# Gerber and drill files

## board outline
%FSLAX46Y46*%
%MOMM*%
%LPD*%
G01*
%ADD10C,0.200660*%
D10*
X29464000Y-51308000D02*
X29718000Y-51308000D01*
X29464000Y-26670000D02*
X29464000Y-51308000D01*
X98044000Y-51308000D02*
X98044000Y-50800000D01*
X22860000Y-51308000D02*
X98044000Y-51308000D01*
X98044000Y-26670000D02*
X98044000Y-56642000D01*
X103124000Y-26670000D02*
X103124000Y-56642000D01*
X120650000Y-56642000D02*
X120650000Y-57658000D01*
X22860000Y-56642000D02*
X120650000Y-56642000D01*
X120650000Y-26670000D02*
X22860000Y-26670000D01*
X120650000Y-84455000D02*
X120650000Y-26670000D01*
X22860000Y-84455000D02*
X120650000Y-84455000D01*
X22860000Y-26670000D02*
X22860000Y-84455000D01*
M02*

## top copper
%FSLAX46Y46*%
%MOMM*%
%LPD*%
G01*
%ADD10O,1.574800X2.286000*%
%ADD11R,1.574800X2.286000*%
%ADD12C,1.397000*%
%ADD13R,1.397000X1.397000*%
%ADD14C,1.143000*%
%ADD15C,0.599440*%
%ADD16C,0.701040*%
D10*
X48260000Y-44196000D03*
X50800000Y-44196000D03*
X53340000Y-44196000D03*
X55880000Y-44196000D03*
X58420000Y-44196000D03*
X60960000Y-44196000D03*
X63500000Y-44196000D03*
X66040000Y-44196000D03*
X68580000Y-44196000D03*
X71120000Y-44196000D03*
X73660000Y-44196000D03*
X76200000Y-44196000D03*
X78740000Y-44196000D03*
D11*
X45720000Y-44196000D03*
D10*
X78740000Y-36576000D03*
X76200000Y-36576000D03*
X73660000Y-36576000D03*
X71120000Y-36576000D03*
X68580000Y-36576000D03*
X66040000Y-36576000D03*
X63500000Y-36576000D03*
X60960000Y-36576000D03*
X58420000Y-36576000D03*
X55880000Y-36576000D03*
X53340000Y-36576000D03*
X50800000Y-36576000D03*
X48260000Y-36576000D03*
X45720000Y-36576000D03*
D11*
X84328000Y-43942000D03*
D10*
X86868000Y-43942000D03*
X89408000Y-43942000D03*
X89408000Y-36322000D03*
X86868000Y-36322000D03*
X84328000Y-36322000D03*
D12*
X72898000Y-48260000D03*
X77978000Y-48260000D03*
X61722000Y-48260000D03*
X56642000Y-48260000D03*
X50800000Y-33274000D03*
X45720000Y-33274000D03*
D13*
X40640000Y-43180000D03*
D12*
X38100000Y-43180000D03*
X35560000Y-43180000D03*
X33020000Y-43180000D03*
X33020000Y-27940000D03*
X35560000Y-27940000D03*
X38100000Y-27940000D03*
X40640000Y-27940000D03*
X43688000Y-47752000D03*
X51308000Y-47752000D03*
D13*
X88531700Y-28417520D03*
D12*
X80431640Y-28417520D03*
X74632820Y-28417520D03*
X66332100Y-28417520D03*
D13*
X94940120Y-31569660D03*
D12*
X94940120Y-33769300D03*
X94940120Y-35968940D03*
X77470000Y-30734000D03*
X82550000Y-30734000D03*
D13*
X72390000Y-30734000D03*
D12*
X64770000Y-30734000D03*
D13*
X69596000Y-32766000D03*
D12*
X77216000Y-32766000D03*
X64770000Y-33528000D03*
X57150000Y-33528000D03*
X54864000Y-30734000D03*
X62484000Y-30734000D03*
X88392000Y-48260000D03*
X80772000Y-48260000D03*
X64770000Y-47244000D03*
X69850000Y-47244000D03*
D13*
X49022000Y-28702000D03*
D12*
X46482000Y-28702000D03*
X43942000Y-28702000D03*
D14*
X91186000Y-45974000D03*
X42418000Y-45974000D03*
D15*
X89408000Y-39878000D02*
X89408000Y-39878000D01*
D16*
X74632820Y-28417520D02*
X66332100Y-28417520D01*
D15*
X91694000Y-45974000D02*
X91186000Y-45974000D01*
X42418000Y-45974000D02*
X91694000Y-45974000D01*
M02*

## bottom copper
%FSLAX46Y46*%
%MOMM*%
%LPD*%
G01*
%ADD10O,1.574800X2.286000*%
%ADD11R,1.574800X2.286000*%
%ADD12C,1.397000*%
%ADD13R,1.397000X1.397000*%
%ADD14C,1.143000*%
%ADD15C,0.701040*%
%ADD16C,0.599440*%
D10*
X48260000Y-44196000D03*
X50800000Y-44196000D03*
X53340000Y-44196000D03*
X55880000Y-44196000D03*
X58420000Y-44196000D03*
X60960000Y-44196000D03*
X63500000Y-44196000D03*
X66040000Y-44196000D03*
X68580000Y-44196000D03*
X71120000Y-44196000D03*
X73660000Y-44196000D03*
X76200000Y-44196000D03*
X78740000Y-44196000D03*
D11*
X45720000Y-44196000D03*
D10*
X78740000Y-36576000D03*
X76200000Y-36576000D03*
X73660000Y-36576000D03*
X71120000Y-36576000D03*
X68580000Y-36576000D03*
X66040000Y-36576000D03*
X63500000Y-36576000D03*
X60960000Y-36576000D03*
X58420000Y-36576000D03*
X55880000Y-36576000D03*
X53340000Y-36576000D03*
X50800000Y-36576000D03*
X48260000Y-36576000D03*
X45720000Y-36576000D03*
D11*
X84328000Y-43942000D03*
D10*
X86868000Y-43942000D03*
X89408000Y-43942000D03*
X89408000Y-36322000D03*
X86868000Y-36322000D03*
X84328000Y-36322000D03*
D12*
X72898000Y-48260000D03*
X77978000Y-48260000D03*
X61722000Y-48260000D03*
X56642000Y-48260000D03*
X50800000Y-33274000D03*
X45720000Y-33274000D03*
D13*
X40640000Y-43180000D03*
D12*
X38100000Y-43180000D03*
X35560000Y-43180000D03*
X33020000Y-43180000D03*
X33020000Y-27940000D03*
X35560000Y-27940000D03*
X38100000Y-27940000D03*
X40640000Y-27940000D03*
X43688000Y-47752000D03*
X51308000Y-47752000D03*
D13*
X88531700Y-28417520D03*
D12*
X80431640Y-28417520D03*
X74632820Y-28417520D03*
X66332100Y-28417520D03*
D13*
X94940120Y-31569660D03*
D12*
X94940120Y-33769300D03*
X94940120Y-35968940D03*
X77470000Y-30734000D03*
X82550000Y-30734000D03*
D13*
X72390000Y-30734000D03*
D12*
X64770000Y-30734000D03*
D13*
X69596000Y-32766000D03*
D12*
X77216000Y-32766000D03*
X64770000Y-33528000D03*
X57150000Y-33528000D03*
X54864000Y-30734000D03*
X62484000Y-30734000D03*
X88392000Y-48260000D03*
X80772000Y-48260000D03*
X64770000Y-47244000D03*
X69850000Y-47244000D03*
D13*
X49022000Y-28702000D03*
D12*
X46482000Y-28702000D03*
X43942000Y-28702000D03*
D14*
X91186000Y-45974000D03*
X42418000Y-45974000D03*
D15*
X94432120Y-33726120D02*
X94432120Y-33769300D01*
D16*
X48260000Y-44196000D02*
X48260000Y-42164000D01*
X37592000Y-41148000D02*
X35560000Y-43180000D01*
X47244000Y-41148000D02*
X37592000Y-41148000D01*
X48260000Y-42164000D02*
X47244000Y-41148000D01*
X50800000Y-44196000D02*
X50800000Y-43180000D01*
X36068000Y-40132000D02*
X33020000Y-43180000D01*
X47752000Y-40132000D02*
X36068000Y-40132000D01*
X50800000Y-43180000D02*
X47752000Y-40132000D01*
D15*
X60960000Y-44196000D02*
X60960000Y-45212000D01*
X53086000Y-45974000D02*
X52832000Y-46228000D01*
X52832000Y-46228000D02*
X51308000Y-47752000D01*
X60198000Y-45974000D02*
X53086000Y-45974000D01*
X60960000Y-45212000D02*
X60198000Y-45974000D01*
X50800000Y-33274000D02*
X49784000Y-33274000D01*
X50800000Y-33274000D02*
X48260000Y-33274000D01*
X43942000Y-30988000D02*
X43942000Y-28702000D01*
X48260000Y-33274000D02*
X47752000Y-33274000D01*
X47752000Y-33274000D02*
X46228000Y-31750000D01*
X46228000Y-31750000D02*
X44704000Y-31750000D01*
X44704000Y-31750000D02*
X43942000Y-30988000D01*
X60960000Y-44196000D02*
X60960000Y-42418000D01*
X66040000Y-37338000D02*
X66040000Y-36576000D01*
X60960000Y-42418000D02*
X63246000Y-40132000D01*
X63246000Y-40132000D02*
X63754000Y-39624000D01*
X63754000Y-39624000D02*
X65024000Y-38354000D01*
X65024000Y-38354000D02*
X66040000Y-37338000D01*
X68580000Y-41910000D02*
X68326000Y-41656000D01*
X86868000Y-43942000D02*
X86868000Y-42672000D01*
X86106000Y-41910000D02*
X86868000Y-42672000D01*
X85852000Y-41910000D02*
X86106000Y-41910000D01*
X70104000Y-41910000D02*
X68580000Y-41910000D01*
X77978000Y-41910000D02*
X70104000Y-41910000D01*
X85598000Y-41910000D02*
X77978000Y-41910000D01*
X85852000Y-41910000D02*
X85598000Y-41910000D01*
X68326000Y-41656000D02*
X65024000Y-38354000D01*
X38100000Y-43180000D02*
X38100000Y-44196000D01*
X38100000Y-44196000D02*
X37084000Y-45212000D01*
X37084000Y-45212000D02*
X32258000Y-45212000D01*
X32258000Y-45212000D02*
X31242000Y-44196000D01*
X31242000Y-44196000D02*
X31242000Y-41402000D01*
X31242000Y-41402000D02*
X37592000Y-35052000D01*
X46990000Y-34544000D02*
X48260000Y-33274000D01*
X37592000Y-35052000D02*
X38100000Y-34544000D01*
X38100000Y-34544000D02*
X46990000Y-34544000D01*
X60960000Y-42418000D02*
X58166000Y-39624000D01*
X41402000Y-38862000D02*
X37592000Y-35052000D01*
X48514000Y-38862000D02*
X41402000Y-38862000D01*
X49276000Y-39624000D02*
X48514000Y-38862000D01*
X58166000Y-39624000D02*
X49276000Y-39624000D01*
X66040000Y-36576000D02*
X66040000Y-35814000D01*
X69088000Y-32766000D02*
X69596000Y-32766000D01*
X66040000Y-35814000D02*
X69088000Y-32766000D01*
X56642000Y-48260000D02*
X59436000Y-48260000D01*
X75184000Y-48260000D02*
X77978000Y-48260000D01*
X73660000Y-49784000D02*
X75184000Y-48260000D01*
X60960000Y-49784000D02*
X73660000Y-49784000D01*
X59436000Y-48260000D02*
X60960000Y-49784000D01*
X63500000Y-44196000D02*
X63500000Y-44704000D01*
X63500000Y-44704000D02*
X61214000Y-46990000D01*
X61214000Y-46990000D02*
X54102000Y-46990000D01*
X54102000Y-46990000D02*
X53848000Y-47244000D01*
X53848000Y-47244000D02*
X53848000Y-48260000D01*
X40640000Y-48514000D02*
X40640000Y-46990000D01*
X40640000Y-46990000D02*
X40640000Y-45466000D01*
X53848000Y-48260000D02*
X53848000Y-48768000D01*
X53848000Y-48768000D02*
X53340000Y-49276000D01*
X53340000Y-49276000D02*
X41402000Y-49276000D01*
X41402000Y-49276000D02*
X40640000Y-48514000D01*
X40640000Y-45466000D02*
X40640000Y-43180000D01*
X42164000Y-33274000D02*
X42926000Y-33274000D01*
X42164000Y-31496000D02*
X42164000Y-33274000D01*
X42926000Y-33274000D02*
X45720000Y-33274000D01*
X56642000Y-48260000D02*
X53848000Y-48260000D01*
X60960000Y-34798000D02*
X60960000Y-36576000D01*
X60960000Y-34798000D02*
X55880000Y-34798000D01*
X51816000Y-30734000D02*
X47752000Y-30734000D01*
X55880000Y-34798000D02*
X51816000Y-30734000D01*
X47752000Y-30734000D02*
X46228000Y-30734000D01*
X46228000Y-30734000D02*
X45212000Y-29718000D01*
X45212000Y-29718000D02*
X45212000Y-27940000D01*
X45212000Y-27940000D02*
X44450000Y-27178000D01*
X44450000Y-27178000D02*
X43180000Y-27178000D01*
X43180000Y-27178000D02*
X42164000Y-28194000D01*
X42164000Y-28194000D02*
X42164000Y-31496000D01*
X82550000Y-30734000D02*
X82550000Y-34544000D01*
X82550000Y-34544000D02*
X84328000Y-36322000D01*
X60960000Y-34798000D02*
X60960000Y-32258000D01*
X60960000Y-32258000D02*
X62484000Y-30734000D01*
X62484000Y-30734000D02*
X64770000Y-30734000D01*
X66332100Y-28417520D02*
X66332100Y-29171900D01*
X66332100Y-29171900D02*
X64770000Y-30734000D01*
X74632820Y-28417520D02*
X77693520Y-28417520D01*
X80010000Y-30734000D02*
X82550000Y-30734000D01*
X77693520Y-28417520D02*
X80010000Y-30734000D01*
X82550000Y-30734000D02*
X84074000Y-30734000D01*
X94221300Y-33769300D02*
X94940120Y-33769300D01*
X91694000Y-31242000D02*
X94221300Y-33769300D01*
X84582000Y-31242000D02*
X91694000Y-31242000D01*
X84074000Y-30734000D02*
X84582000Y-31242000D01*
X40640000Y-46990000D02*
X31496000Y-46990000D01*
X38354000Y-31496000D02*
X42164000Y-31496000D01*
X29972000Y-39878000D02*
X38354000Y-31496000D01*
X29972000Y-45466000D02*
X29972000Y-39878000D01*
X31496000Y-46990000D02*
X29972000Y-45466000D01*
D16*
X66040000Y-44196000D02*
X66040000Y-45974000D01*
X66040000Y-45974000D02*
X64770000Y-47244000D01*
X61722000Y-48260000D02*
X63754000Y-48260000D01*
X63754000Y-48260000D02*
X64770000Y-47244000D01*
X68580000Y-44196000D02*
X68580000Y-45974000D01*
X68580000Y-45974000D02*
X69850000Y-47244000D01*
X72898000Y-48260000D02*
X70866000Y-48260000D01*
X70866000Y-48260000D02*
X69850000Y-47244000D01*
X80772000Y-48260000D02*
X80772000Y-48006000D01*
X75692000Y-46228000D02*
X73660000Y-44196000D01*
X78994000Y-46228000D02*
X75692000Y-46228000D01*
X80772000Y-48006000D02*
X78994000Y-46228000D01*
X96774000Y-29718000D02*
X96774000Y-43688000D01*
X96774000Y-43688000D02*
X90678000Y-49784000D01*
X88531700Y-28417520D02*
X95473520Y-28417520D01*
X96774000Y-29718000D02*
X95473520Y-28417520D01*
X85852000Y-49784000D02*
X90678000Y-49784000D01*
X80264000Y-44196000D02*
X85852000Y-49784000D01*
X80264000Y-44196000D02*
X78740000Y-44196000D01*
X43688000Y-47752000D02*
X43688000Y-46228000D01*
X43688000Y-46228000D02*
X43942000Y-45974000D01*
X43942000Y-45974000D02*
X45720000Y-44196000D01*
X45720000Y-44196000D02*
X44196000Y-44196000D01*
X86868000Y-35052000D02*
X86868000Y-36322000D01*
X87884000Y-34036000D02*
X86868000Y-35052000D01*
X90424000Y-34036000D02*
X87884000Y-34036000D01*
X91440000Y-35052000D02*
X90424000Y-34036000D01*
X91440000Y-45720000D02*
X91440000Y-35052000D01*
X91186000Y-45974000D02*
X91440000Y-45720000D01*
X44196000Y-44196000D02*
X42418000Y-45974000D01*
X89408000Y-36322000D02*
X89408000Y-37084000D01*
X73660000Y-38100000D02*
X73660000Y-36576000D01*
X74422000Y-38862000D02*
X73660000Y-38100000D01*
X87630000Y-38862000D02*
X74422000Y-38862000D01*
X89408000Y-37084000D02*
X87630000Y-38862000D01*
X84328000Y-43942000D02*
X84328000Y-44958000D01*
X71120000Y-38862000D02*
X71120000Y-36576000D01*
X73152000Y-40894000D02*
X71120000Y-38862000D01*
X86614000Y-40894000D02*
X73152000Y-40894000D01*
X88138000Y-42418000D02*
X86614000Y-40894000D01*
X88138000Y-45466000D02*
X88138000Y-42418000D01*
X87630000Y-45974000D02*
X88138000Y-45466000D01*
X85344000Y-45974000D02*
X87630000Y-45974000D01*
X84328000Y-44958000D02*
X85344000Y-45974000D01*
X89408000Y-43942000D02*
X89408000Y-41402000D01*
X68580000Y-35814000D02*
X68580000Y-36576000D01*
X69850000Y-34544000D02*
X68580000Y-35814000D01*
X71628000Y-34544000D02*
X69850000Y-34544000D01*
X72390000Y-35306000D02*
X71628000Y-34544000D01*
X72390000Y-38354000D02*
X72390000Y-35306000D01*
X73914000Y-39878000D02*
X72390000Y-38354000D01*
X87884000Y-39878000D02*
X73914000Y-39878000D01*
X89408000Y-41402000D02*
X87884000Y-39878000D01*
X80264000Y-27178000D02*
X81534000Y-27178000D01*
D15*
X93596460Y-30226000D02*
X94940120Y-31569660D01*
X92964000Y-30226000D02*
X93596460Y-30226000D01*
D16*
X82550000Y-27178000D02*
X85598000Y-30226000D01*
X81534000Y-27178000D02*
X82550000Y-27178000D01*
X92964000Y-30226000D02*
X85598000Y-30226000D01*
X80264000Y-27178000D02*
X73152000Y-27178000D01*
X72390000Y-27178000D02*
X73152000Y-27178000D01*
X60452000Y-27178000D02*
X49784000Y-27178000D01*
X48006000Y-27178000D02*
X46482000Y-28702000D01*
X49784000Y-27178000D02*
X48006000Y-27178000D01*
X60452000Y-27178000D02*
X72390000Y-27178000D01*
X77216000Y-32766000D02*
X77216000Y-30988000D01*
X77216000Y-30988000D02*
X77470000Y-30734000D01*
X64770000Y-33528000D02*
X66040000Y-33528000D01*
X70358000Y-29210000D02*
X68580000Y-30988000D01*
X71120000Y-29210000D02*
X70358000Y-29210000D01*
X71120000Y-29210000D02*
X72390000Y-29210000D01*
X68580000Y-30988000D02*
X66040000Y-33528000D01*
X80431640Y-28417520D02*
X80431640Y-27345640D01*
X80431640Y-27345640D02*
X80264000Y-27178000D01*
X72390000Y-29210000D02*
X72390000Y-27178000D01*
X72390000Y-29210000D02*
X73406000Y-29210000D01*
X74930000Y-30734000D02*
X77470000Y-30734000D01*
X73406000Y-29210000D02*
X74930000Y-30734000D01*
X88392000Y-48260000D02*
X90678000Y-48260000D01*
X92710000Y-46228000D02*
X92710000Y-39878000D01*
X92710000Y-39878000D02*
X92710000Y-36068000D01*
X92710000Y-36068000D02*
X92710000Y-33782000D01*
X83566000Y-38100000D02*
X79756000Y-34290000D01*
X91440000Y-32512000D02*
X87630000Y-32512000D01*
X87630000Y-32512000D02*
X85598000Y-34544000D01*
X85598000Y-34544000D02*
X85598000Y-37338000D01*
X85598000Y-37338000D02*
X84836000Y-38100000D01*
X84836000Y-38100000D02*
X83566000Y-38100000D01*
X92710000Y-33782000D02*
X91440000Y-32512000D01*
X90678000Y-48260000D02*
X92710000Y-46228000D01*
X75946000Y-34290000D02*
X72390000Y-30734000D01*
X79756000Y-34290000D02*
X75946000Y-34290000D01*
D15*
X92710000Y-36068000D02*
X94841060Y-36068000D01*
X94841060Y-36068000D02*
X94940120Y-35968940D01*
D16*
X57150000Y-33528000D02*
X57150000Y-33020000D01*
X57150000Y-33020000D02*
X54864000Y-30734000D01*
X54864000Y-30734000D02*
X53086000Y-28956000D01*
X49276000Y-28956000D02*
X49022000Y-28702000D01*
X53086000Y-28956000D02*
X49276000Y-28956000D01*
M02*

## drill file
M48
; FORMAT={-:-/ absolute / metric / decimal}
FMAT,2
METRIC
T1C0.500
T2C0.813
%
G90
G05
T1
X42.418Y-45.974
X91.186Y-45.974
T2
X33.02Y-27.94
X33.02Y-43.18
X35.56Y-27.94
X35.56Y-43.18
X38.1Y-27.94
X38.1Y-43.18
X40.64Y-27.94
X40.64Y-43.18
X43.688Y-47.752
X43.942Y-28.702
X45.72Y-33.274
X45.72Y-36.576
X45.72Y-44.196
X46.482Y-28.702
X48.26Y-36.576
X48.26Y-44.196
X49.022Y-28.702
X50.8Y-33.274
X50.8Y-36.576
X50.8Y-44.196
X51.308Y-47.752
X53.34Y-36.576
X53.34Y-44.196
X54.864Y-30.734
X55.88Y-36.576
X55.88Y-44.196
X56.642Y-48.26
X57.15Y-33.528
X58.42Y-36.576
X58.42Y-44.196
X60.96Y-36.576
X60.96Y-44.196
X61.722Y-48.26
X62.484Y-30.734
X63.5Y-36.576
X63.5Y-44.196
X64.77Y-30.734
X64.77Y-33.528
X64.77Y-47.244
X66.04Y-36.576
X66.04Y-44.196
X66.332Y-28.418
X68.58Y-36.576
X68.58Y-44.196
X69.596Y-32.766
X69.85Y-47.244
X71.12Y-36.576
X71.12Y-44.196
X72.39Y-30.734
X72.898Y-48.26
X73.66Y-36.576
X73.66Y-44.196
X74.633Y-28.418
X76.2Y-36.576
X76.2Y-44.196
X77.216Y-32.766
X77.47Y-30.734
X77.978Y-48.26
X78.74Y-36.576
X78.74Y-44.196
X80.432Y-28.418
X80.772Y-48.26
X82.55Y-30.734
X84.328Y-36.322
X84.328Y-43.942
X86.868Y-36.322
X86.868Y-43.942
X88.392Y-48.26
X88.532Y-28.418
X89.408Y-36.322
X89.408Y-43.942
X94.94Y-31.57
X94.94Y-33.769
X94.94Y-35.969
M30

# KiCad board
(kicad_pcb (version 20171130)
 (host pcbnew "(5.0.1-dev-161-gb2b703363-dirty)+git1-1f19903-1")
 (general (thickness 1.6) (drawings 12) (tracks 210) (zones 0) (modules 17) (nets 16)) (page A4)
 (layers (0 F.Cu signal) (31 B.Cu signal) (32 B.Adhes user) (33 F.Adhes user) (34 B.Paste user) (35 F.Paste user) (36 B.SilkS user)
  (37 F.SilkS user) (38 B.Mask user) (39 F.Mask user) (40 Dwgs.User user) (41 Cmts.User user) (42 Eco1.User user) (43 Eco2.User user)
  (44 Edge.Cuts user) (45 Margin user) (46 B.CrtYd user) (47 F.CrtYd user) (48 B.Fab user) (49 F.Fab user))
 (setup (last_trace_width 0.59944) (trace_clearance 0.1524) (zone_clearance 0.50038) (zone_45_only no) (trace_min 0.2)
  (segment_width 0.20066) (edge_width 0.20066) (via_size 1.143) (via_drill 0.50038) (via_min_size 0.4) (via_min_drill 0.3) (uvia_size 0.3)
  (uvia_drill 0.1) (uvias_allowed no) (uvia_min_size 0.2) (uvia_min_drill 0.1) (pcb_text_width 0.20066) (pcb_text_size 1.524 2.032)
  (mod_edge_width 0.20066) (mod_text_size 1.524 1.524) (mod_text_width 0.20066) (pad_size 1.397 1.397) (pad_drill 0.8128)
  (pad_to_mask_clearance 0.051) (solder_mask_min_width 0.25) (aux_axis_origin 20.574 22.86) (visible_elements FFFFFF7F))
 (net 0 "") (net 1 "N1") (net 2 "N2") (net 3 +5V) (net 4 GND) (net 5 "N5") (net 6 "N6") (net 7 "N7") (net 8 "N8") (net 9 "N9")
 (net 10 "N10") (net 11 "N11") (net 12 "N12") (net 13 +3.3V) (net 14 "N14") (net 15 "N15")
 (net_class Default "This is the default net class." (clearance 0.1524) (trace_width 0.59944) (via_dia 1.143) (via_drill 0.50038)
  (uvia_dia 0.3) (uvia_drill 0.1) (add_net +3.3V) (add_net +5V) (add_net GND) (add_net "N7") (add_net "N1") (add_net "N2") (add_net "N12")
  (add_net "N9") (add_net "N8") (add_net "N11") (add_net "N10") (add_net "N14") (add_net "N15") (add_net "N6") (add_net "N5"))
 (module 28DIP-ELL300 (layer F.Cu) (at 62.23 40.386)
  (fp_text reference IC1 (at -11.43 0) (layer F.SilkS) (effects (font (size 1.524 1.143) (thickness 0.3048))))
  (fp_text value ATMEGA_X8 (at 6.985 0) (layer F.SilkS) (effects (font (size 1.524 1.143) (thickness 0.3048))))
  (pad 2 thru_hole oval (at -13.97 3.81) (size 1.5748 2.286) (drill 0.8128) (layers *.Cu *.Mask F.SilkS) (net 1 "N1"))
  (pad 3 thru_hole oval (at -11.43 3.81) (size 1.5748 2.286) (drill 0.8128) (layers *.Cu *.Mask F.SilkS) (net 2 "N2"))
  (pad 4 thru_hole oval (at -8.89 3.81) (size 1.5748 2.286) (drill 0.8128) (layers *.Cu *.Mask F.SilkS))
  (pad 5 thru_hole oval (at -6.35 3.81) (size 1.5748 2.286) (drill 0.8128) (layers *.Cu *.Mask F.SilkS))
  (pad 6 thru_hole oval (at -3.81 3.81) (size 1.5748 2.286) (drill 0.8128) (layers *.Cu *.Mask F.SilkS))
  (pad 7 thru_hole oval (at -1.27 3.81) (size 1.5748 2.286) (drill 0.8128) (layers *.Cu *.Mask F.SilkS) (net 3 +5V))
  (pad 8 thru_hole oval (at 1.27 3.81) (size 1.5748 2.286) (drill 0.8128) (layers *.Cu *.Mask F.SilkS) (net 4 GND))
  (pad 9 thru_hole oval (at 3.81 3.81) (size 1.5748 2.286) (drill 0.8128) (layers *.Cu *.Mask F.SilkS) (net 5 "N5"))
  (pad 10 thru_hole oval (at 6.35 3.81) (size 1.5748 2.286) (drill 0.8128) (layers *.Cu *.Mask F.SilkS) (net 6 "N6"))
  (pad 11 thru_hole oval (at 8.89 3.81) (size 1.5748 2.286) (drill 0.8128) (layers *.Cu *.Mask F.SilkS))
  (pad 12 thru_hole oval (at 11.43 3.81) (size 1.5748 2.286) (drill 0.8128) (layers *.Cu *.Mask F.SilkS) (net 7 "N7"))
  (pad 13 thru_hole oval (at 13.97 3.81) (size 1.5748 2.286) (drill 0.8128) (layers *.Cu *.Mask F.SilkS))
  (pad 14 thru_hole oval (at 16.51 3.81) (size 1.5748 2.286) (drill 0.8128) (layers *.Cu *.Mask F.SilkS) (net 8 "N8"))
  (pad 1 thru_hole rect (at -16.51 3.81) (size 1.5748 2.286) (drill 0.8128) (layers *.Cu *.Mask F.SilkS) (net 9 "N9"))
  (pad 15 thru_hole oval (at 16.51 -3.81) (size 1.5748 2.286) (drill 0.8128) (layers *.Cu *.Mask F.SilkS))
  (pad 16 thru_hole oval (at 13.97 -3.81) (size 1.5748 2.286) (drill 0.8128) (layers *.Cu *.Mask F.SilkS))
  (pad 17 thru_hole oval (at 11.43 -3.81) (size 1.5748 2.286) (drill 0.8128) (layers *.Cu *.Mask F.SilkS) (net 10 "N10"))
  (pad 18 thru_hole oval (at 8.89 -3.81) (size 1.5748 2.286) (drill 0.8128) (layers *.Cu *.Mask F.SilkS) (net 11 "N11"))
  (pad 19 thru_hole oval (at 6.35 -3.81) (size 1.5748 2.286) (drill 0.8128) (layers *.Cu *.Mask F.SilkS) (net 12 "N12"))
  (pad 20 thru_hole oval (at 3.81 -3.81) (size 1.5748 2.286) (drill 0.8128) (layers *.Cu *.Mask F.SilkS) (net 3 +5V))
  (pad 21 thru_hole oval (at 1.27 -3.81) (size 1.5748 2.286) (drill 0.8128) (layers *.Cu *.Mask F.SilkS))
  (pad 22 thru_hole oval (at -1.27 -3.81) (size 1.5748 2.286) (drill 0.8128) (layers *.Cu *.Mask F.SilkS) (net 4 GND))
  (pad 23 thru_hole oval (at -3.81 -3.81) (size 1.5748 2.286) (drill 0.8128) (layers *.Cu *.Mask F.SilkS))
  (pad 24 thru_hole oval (at -6.35 -3.81) (size 1.5748 2.286) (drill 0.8128) (layers *.Cu *.Mask F.SilkS))
  (pad 25 thru_hole oval (at -8.89 -3.81) (size 1.5748 2.286) (drill 0.8128) (layers *.Cu *.Mask F.SilkS))
  (pad 26 thru_hole oval (at -11.43 -3.81) (size 1.5748 2.286) (drill 0.8128) (layers *.Cu *.Mask F.SilkS))
  (pad 27 thru_hole oval (at -13.97 -3.81) (size 1.5748 2.286) (drill 0.8128) (layers *.Cu *.Mask F.SilkS))
  (pad 28 thru_hole oval (at -16.51 -3.81) (size 1.5748 2.286) (drill 0.8128) (layers *.Cu *.Mask F.SilkS)))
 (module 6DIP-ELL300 (layer F.Cu) (at 86.868 40.132)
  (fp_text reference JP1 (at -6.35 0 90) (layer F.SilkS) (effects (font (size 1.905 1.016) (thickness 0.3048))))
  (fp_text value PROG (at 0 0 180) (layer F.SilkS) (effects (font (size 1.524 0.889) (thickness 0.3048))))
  (pad 1 thru_hole rect (at -2.54 3.81) (size 1.5748 2.286) (drill 0.8128) (layers *.Cu *.Mask F.SilkS) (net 11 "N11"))
  (pad 2 thru_hole oval (at 0 3.81) (size 1.5748 2.286) (drill 0.8128) (layers *.Cu *.Mask F.SilkS) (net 3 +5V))
  (pad 3 thru_hole oval (at 2.54 3.81) (size 1.5748 2.286) (drill 0.8128) (layers *.Cu *.Mask F.SilkS) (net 12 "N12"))
  (pad 4 thru_hole oval (at 2.54 -3.81) (size 1.5748 2.286) (drill 0.8128) (layers *.Cu *.Mask F.SilkS) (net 10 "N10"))
  (pad 5 thru_hole oval (at 0 -3.81) (size 1.5748 2.286) (drill 0.8128) (layers *.Cu *.Mask F.SilkS) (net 9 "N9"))
  (pad 6 thru_hole oval (at -2.54 -3.81) (size 1.5748 2.286) (drill 0.8128) (layers *.Cu *.Mask F.SilkS) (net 4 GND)))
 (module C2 (layer F.Cu) (at 75.438 48.26)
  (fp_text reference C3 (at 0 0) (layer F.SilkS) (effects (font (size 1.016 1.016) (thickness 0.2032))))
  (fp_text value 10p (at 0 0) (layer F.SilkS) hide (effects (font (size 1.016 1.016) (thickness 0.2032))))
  (pad 1 thru_hole circle (at -2.54 0) (size 1.397 1.397) (drill 0.8128) (layers *.Cu *.Mask F.SilkS) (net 6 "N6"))
  (pad 2 thru_hole circle (at 2.54 0) (size 1.397 1.397) (drill 0.8128) (layers *.Cu *.Mask F.SilkS) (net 4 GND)))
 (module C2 (layer F.Cu) (at 59.182 48.26 180)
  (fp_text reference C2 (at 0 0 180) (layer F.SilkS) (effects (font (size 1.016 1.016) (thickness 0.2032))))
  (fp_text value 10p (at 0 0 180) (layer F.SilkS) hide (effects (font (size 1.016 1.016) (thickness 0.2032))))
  (pad 1 thru_hole circle (at -2.54 0 180) (size 1.397 1.397) (drill 0.8128) (layers *.Cu *.Mask F.SilkS) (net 5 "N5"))
  (pad 2 thru_hole circle (at 2.54 0 180) (size 1.397 1.397) (drill 0.8128) (layers *.Cu *.Mask F.SilkS) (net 4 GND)))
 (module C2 (layer F.Cu) (at 48.26 33.274 180)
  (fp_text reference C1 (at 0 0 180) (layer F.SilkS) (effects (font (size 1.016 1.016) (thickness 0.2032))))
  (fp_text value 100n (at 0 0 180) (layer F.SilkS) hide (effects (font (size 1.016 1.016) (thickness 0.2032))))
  (pad 1 thru_hole circle (at -2.54 0 180) (size 1.397 1.397) (drill 0.8128) (layers *.Cu *.Mask F.SilkS) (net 3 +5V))
  (pad 2 thru_hole circle (at 2.54 0 180) (size 1.397 1.397) (drill 0.8128) (layers *.Cu *.Mask F.SilkS) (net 4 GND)))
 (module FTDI (layer F.Cu) (at 41.91 26.67 270)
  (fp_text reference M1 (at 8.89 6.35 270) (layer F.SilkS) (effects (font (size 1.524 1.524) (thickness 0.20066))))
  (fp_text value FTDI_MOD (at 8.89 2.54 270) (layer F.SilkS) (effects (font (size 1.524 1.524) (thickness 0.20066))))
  (pad 1 thru_hole rect (at 16.51 1.27 270) (size 1.397 1.397) (drill 0.8128) (layers *.Cu *.Mask F.SilkS) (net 4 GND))
  (pad 2 thru_hole circle (at 16.51 3.81 270) (size 1.397 1.397) (drill 0.8128) (layers *.Cu *.Mask F.SilkS) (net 3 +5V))
  (pad 3 thru_hole circle (at 16.51 6.35 270) (size 1.397 1.397) (drill 0.8128) (layers *.Cu *.Mask F.SilkS) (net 1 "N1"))
  (pad 4 thru_hole circle (at 16.51 8.89 270) (size 1.397 1.397) (drill 0.8128) (layers *.Cu *.Mask F.SilkS) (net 2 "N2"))
  (pad 8 thru_hole circle (at 1.27 8.89 270) (size 1.397 1.397) (drill 0.8128) (layers *.Cu *.Mask F.SilkS))
  (pad 7 thru_hole circle (at 1.27 6.35 270) (size 1.397 1.397) (drill 0.8128) (layers *.Cu *.Mask F.SilkS))
  (pad 6 thru_hole circle (at 1.27 3.81 270) (size 1.397 1.397) (drill 0.8128) (layers *.Cu *.Mask F.SilkS))
  (pad 5 thru_hole circle (at 1.27 1.27 270) (size 1.397 1.397) (drill 0.8128) (layers *.Cu *.Mask F.SilkS)))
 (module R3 (layer F.Cu) (at 47.498 47.752) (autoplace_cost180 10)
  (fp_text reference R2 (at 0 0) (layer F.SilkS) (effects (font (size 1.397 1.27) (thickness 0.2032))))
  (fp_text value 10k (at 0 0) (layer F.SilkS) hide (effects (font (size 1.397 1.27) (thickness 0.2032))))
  (pad 1 thru_hole circle (at -3.81 0) (size 1.397 1.397) (drill 0.8128) (layers *.Cu *.Mask F.SilkS) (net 9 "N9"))
  (pad 2 thru_hole circle (at 3.81 0) (size 1.397 1.397) (drill 0.8128) (layers *.Cu *.Mask F.SilkS) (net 3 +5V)))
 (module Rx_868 (layer F.Cu) (at 90.932 29.718 180)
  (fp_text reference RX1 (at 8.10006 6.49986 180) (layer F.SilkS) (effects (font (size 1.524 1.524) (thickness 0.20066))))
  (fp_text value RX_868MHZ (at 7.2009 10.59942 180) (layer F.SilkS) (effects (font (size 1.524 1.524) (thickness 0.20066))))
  (pad 1 thru_hole rect (at 2.4003 1.30048 180) (size 1.397 1.397) (drill 0.8128) (layers *.Cu *.Mask F.SilkS) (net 8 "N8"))
  (pad 2 thru_hole circle (at 10.50036 1.30048 180) (size 1.397 1.397) (drill 0.8128) (layers *.Cu *.Mask F.SilkS) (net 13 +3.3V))
  (pad 3 thru_hole circle (at 16.29918 1.30048 180) (size 1.397 1.397) (drill 0.8128) (layers *.Cu *.Mask F.SilkS) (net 4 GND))
  (pad 4 thru_hole circle (at 24.5999 1.30048 180) (size 1.397 1.397) (drill 0.8128) (layers *.Cu *.Mask F.SilkS) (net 4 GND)))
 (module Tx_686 (layer F.Cu) (at 91.44 26.67 270)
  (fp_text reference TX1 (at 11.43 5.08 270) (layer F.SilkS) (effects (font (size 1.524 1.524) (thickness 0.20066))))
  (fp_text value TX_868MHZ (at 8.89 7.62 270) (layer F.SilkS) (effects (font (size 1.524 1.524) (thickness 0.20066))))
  (pad 1 thru_hole rect (at 4.89966 -3.50012 270) (size 1.397 1.397) (drill 0.8128) (layers *.Cu *.Mask F.SilkS) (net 13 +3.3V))
  (pad 2 thru_hole circle (at 7.0993 -3.50012 270) (size 1.397 1.397) (drill 0.8128) (layers *.Cu *.Mask F.SilkS) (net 4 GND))
  (pad 3 thru_hole circle (at 9.29894 -3.50012 270) (size 1.397 1.397) (drill 0.8128) (layers *.Cu *.Mask F.SilkS) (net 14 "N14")))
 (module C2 (layer F.Cu) (at 80.01 30.734)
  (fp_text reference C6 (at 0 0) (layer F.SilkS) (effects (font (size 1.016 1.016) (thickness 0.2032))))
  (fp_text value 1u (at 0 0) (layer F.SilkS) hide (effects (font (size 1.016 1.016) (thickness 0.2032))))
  (pad 1 thru_hole circle (at -2.54 0) (size 1.397 1.397) (drill 0.8128) (layers *.Cu *.Mask F.SilkS) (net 13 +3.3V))
  (pad 2 thru_hole circle (at 2.54 0) (size 1.397 1.397) (drill 0.8128) (layers *.Cu *.Mask F.SilkS) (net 4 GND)))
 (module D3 (layer F.Cu) (at 68.58 30.734)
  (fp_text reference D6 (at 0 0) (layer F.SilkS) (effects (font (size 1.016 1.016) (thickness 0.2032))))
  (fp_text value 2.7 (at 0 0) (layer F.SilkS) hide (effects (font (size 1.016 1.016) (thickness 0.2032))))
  (pad 2 thru_hole rect (at 3.81 0) (size 1.397 1.397) (drill 0.8128) (layers *.Cu *.Mask F.SilkS) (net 14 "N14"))
  (pad 1 thru_hole circle (at -3.81 0) (size 1.397 1.397) (drill 0.8128) (layers *.Cu *.Mask F.SilkS) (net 4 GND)))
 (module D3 (layer F.Cu) (at 73.406 32.766 180)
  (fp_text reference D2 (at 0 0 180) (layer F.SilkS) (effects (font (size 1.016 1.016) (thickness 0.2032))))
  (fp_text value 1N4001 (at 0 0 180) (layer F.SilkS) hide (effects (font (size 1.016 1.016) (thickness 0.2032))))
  (pad 2 thru_hole rect (at 3.81 0 180) (size 1.397 1.397) (drill 0.8128) (layers *.Cu *.Mask F.SilkS) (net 3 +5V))
  (pad 1 thru_hole circle (at -3.81 0 180) (size 1.397 1.397) (drill 0.8128) (layers *.Cu *.Mask F.SilkS) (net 13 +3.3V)))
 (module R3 (layer F.Cu) (at 60.96 33.528 180) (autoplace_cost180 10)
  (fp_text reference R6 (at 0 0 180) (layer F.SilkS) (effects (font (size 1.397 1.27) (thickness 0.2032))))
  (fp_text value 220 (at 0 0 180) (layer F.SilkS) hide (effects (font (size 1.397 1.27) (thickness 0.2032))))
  (pad 1 thru_hole circle (at -3.81 0 180) (size 1.397 1.397) (drill 0.8128) (layers *.Cu *.Mask F.SilkS) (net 13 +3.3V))
  (pad 2 thru_hole circle (at 3.81 0 180) (size 1.397 1.397) (drill 0.8128) (layers *.Cu *.Mask F.SilkS) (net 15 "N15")))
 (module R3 (layer F.Cu) (at 58.674 30.734) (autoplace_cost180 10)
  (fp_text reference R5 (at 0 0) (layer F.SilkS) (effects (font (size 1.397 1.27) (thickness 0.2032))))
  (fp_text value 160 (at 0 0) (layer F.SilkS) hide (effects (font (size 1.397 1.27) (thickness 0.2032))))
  (pad 1 thru_hole circle (at -3.81 0) (size 1.397 1.397) (drill 0.8128) (layers *.Cu *.Mask F.SilkS) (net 15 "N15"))
  (pad 2 thru_hole circle (at 3.81 0) (size 1.397 1.397) (drill 0.8128) (layers *.Cu *.Mask F.SilkS) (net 4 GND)))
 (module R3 (layer F.Cu) (at 84.582 48.26 180) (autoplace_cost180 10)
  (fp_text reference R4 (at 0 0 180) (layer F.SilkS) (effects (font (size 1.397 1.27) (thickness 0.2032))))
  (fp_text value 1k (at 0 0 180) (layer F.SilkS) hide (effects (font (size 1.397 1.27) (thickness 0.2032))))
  (pad 1 thru_hole circle (at -3.81 0 180) (size 1.397 1.397) (drill 0.8128) (layers *.Cu *.Mask F.SilkS) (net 14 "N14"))
  (pad 2 thru_hole circle (at 3.81 0 180) (size 1.397 1.397) (drill 0.8128) (layers *.Cu *.Mask F.SilkS) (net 7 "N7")))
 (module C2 (layer F.Cu) (at 67.31 47.244)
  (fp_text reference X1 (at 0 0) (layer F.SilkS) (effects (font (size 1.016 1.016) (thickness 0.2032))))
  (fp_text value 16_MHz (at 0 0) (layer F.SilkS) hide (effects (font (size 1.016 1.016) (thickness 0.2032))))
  (pad 1 thru_hole circle (at -2.54 0) (size 1.397 1.397) (drill 0.8128) (layers *.Cu *.Mask F.SilkS) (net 5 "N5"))
  (pad 2 thru_hole circle (at 2.54 0) (size 1.397 1.397) (drill 0.8128) (layers *.Cu *.Mask F.SilkS) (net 6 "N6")))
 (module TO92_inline (layer F.Cu) (at 46.482 28.702 180)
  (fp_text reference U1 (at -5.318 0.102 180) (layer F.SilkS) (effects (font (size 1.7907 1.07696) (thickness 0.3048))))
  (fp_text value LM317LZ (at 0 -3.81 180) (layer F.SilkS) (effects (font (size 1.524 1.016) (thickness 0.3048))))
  (pad 1 thru_hole rect (at -2.54 0 180) (size 1.397 1.397) (drill 0.8128) (layers *.Cu *.Mask F.SilkS) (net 15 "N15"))
  (pad 2 thru_hole circle (at 0 0 180) (size 1.397 1.397) (drill 0.8128) (layers *.Cu *.Mask F.SilkS) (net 13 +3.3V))
  (pad 3 thru_hole circle (at 2.54 0 180) (size 1.397 1.397) (drill 0.8128) (layers *.Cu *.Mask F.SilkS) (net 3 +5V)))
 (gr_line (start 29.464 51.308) (end 29.718 51.308) (angle 90) (layer Edge.Cuts) (width 0.20066))
 (gr_line (start 29.464 26.67) (end 29.464 51.308) (angle 90) (layer Edge.Cuts) (width 0.20066))
 (gr_line (start 98.044 51.308) (end 98.044 50.8) (angle 90) (layer Edge.Cuts) (width 0.20066))
 (gr_line (start 22.86 51.308) (end 98.044 51.308) (angle 90) (layer Edge.Cuts) (width 0.20066))
 (gr_line (start 98.044 26.67) (end 98.044 56.642) (angle 90) (layer Edge.Cuts) (width 0.20066))
 (gr_line (start 103.124 26.67) (end 103.124 56.642) (angle 90) (layer Edge.Cuts) (width 0.20066))
 (gr_line (start 120.65 56.642) (end 120.65 57.658) (angle 90) (layer Edge.Cuts) (width 0.20066))
 (gr_line (start 22.86 56.642) (end 120.65 56.642) (angle 90) (layer Edge.Cuts) (width 0.20066))
 (gr_line (start 120.65 26.67) (end 22.86 26.67) (angle 90) (layer Edge.Cuts) (width 0.20066))
 (gr_line (start 120.65 84.455) (end 120.65 26.67) (angle 90) (layer Edge.Cuts) (width 0.20066))
 (gr_line (start 22.86 84.455) (end 120.65 84.455) (angle 90) (layer Edge.Cuts) (width 0.20066))
 (gr_line (start 22.86 26.67) (end 22.86 84.455) (angle 90) (layer Edge.Cuts) (width 0.20066))
 (segment (start 89.408 39.878) (end 89.408 39.878) (width 0.59944) (layer F.Cu) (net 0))
 (segment (start 94.43212 33.72612) (end 94.43212 33.7693) (width 0.70104) (layer B.Cu) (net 4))
 (segment (start 48.26 44.196) (end 48.26 42.164) (width 0.59944) (layer B.Cu) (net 1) (status 800))
 (segment (start 37.592 41.148) (end 35.56 43.18) (width 0.59944) (layer B.Cu) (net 1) (status 400))
 (segment (start 47.244 41.148) (end 37.592 41.148) (width 0.59944) (layer B.Cu) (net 1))
 (segment (start 48.26 42.164) (end 47.244 41.148) (width 0.59944) (layer B.Cu) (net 1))
 (segment (start 50.8 44.196) (end 50.8 43.18) (width 0.59944) (layer B.Cu) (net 2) (status 800))
 (segment (start 36.068 40.132) (end 33.02 43.18) (width 0.59944) (layer B.Cu) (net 2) (status 400))
 (segment (start 47.752 40.132) (end 36.068 40.132) (width 0.59944) (layer B.Cu) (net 2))
 (segment (start 50.8 43.18) (end 47.752 40.132) (width 0.59944) (layer B.Cu) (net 2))
 (segment (start 60.96 44.196) (end 60.96 45.212) (width 0.70104) (layer B.Cu) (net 3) (status 800))
 (segment (start 53.086 45.974) (end 52.832 46.228) (width 0.70104) (layer B.Cu) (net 3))
 (segment (start 52.832 46.228) (end 51.308 47.752) (width 0.70104) (layer B.Cu) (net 3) (status 400))
 (segment (start 60.198 45.974) (end 53.086 45.974) (width 0.70104) (layer B.Cu) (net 3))
 (segment (start 60.96 45.212) (end 60.198 45.974) (width 0.70104) (layer B.Cu) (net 3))
 (segment (start 50.8 33.274) (end 49.784 33.274) (width 0.70104) (layer B.Cu) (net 3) (status 800))
 (segment (start 50.8 33.274) (end 48.26 33.274) (width 0.70104) (layer B.Cu) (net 3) (status 800))
 (segment (start 43.942 30.988) (end 43.942 28.702) (width 0.70104) (layer B.Cu) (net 3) (status 400))
 (segment (start 48.26 33.274) (end 47.752 33.274) (width 0.70104) (layer B.Cu) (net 3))
 (segment (start 47.752 33.274) (end 46.228 31.75) (width 0.70104) (layer B.Cu) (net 3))
 (segment (start 46.228 31.75) (end 44.704 31.75) (width 0.70104) (layer B.Cu) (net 3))
 (segment (start 44.704 31.75) (end 43.942 30.988) (width 0.70104) (layer B.Cu) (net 3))
 (segment (start 60.96 44.196) (end 60.96 42.418) (width 0.70104) (layer B.Cu) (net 3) (status 800))
 (segment (start 66.04 37.338) (end 66.04 36.576) (width 0.70104) (layer B.Cu) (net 3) (status 400))
 (segment (start 60.96 42.418) (end 63.246 40.132) (width 0.70104) (layer B.Cu) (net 3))
 (segment (start 63.246 40.132) (end 63.754 39.624) (width 0.70104) (layer B.Cu) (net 3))
 (segment (start 63.754 39.624) (end 65.024 38.354) (width 0.70104) (layer B.Cu) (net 3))
 (segment (start 65.024 38.354) (end 66.04 37.338) (width 0.70104) (layer B.Cu) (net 3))
 (segment (start 68.58 41.91) (end 68.326 41.656) (width 0.70104) (layer B.Cu) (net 3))
 (segment (start 86.868 43.942) (end 86.868 42.672) (width 0.70104) (layer B.Cu) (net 3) (status 800))
 (segment (start 86.106 41.91) (end 86.868 42.672) (width 0.70104) (layer B.Cu) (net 3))
 (segment (start 85.852 41.91) (end 86.106 41.91) (width 0.70104) (layer B.Cu) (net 3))
 (segment (start 70.104 41.91) (end 68.58 41.91) (width 0.70104) (layer B.Cu) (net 3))
 (segment (start 77.978 41.91) (end 70.104 41.91) (width 0.70104) (layer B.Cu) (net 3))
 (segment (start 85.598 41.91) (end 77.978 41.91) (width 0.70104) (layer B.Cu) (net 3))
 (segment (start 85.852 41.91) (end 85.598 41.91) (width 0.70104) (layer B.Cu) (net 3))
 (segment (start 68.326 41.656) (end 65.024 38.354) (width 0.70104) (layer B.Cu) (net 3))
 (segment (start 38.1 43.18) (end 38.1 44.196) (width 0.70104) (layer B.Cu) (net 3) (status 800))
 (segment (start 38.1 44.196) (end 37.084 45.212) (width 0.70104) (layer B.Cu) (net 3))
 (segment (start 37.084 45.212) (end 32.258 45.212) (width 0.70104) (layer B.Cu) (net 3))
 (segment (start 32.258 45.212) (end 31.242 44.196) (width 0.70104) (layer B.Cu) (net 3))
 (segment (start 31.242 44.196) (end 31.242 41.402) (width 0.70104) (layer B.Cu) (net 3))
 (segment (start 31.242 41.402) (end 37.592 35.052) (width 0.70104) (layer B.Cu) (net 3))
 (segment (start 46.99 34.544) (end 48.26 33.274) (width 0.70104) (layer B.Cu) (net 3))
 (segment (start 37.592 35.052) (end 38.1 34.544) (width 0.70104) (layer B.Cu) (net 3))
 (segment (start 38.1 34.544) (end 46.99 34.544) (width 0.70104) (layer B.Cu) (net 3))
 (segment (start 60.96 42.418) (end 58.166 39.624) (width 0.70104) (layer B.Cu) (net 3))
 (segment (start 41.402 38.862) (end 37.592 35.052) (width 0.70104) (layer B.Cu) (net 3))
 (segment (start 48.514 38.862) (end 41.402 38.862) (width 0.70104) (layer B.Cu) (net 3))
 (segment (start 49.276 39.624) (end 48.514 38.862) (width 0.70104) (layer B.Cu) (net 3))
 (segment (start 58.166 39.624) (end 49.276 39.624) (width 0.70104) (layer B.Cu) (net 3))
 (segment (start 66.04 36.576) (end 66.04 35.814) (width 0.70104) (layer B.Cu) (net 3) (status C00))
 (segment (start 69.088 32.766) (end 69.596 32.766) (width 0.70104) (layer B.Cu) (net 3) (status C00))
 (segment (start 66.04 35.814) (end 69.088 32.766) (width 0.70104) (layer B.Cu) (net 3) (status C00))
 (segment (start 56.642 48.26) (end 59.436 48.26) (width 0.70104) (layer B.Cu) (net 4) (status 800))
 (segment (start 75.184 48.26) (end 77.978 48.26) (width 0.70104) (layer B.Cu) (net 4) (status 400))
 (segment (start 73.66 49.784) (end 75.184 48.26) (width 0.70104) (layer B.Cu) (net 4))
 (segment (start 60.96 49.784) (end 73.66 49.784) (width 0.70104) (layer B.Cu) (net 4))
 (segment (start 59.436 48.26) (end 60.96 49.784) (width 0.70104) (layer B.Cu) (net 4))
 (segment (start 63.5 44.196) (end 63.5 44.704) (width 0.70104) (layer B.Cu) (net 4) (status 800))
 (segment (start 63.5 44.704) (end 61.214 46.99) (width 0.70104) (layer B.Cu) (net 4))
 (segment (start 61.214 46.99) (end 54.102 46.99) (width 0.70104) (layer B.Cu) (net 4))
 (segment (start 54.102 46.99) (end 53.848 47.244) (width 0.70104) (layer B.Cu) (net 4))
 (segment (start 53.848 47.244) (end 53.848 48.26) (width 0.70104) (layer B.Cu) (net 4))
 (segment (start 40.64 48.514) (end 40.64 46.99) (width 0.70104) (layer B.Cu) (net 4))
 (segment (start 40.64 46.99) (end 40.64 45.466) (width 0.70104) (layer B.Cu) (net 4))
 (segment (start 53.848 48.26) (end 53.848 48.768) (width 0.70104) (layer B.Cu) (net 4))
 (segment (start 53.848 48.768) (end 53.34 49.276) (width 0.70104) (layer B.Cu) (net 4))
 (segment (start 53.34 49.276) (end 41.402 49.276) (width 0.70104) (layer B.Cu) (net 4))
 (segment (start 41.402 49.276) (end 40.64 48.514) (width 0.70104) (layer B.Cu) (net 4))
 (segment (start 40.64 45.466) (end 40.64 43.18) (width 0.70104) (layer B.Cu) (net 4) (status 400))
 (segment (start 42.164 33.274) (end 42.926 33.274) (width 0.70104) (layer B.Cu) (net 4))
 (segment (start 42.164 31.496) (end 42.164 33.274) (width 0.70104) (layer B.Cu) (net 4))
 (segment (start 42.926 33.274) (end 45.72 33.274) (width 0.70104) (layer B.Cu) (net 4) (status 400))
 (segment (start 56.642 48.26) (end 53.848 48.26) (width 0.70104) (layer B.Cu) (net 4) (status 800))
 (segment (start 60.96 34.798) (end 60.96 36.576) (width 0.70104) (layer B.Cu) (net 4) (status 400))
 (segment (start 60.96 34.798) (end 55.88 34.798) (width 0.70104) (layer B.Cu) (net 4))
 (segment (start 51.816 30.734) (end 47.752 30.734) (width 0.70104) (layer B.Cu) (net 4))
 (segment (start 55.88 34.798) (end 51.816 30.734) (width 0.70104) (layer B.Cu) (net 4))
 (segment (start 47.752 30.734) (end 46.228 30.734) (width 0.70104) (layer B.Cu) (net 4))
 (segment (start 46.228 30.734) (end 45.212 29.718) (width 0.70104) (layer B.Cu) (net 4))
 (segment (start 45.212 29.718) (end 45.212 27.94) (width 0.70104) (layer B.Cu) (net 4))
 (segment (start 45.212 27.94) (end 44.45 27.178) (width 0.70104) (layer B.Cu) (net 4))
 (segment (start 44.45 27.178) (end 43.18 27.178) (width 0.70104) (layer B.Cu) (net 4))
 (segment (start 43.18 27.178) (end 42.164 28.194) (width 0.70104) (layer B.Cu) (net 4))
 (segment (start 42.164 28.194) (end 42.164 31.496) (width 0.70104) (layer B.Cu) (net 4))
 (segment (start 82.55 30.734) (end 82.55 34.544) (width 0.70104) (layer B.Cu) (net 4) (status 800))
 (segment (start 82.55 34.544) (end 84.328 36.322) (width 0.70104) (layer B.Cu) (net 4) (status 400))
 (segment (start 60.96 34.798) (end 60.96 32.258) (width 0.70104) (layer B.Cu) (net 4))
 (segment (start 60.96 32.258) (end 62.484 30.734) (width 0.70104) (layer B.Cu) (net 4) (status 400))
 (segment (start 62.484 30.734) (end 64.77 30.734) (width 0.70104) (layer B.Cu) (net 4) (status C00))
 (segment (start 74.63282 28.41752) (end 66.3321 28.41752) (width 0.70104) (layer F.Cu) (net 4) (status C00))
 (segment (start 66.3321 28.41752) (end 66.3321 29.1719) (width 0.70104) (layer B.Cu) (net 4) (status 800))
 (segment (start 66.3321 29.1719) (end 64.77 30.734) (width 0.70104) (layer B.Cu) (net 4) (status 400))
 (segment (start 74.63282 28.41752) (end 77.69352 28.41752) (width 0.70104) (layer B.Cu) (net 4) (status 800))
 (segment (start 80.01 30.734) (end 82.55 30.734) (width 0.70104) (layer B.Cu) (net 4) (status 400))
 (segment (start 77.69352 28.41752) (end 80.01 30.734) (width 0.70104) (layer B.Cu) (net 4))
 (segment (start 82.55 30.734) (end 84.074 30.734) (width 0.70104) (layer B.Cu) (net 4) (status 800))
 (segment (start 94.2213 33.7693) (end 94.94012 33.7693) (width 0.70104) (layer B.Cu) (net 4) (status 400))
 (segment (start 91.694 31.242) (end 94.2213 33.7693) (width 0.70104) (layer B.Cu) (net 4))
 (segment (start 84.582 31.242) (end 91.694 31.242) (width 0.70104) (layer B.Cu) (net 4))
 (segment (start 84.074 30.734) (end 84.582 31.242) (width 0.70104) (layer B.Cu) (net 4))
 (segment (start 40.64 46.99) (end 31.496 46.99) (width 0.70104) (layer B.Cu) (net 4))
 (segment (start 38.354 31.496) (end 42.164 31.496) (width 0.70104) (layer B.Cu) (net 4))
 (segment (start 29.972 39.878) (end 38.354 31.496) (width 0.70104) (layer B.Cu) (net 4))
 (segment (start 29.972 45.466) (end 29.972 39.878) (width 0.70104) (layer B.Cu) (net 4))
 (segment (start 31.496 46.99) (end 29.972 45.466) (width 0.70104) (layer B.Cu) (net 4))
 (segment (start 66.04 44.196) (end 66.04 45.974) (width 0.59944) (layer B.Cu) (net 5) (status 800))
 (segment (start 66.04 45.974) (end 64.77 47.244) (width 0.59944) (layer B.Cu) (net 5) (status 400))
 (segment (start 61.722 48.26) (end 63.754 48.26) (width 0.59944) (layer B.Cu) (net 5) (status 800))
 (segment (start 63.754 48.26) (end 64.77 47.244) (width 0.59944) (layer B.Cu) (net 5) (status 400))
 (segment (start 68.58 44.196) (end 68.58 45.974) (width 0.59944) (layer B.Cu) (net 6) (status 800))
 (segment (start 68.58 45.974) (end 69.85 47.244) (width 0.59944) (layer B.Cu) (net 6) (status 400))
 (segment (start 72.898 48.26) (end 70.866 48.26) (width 0.59944) (layer B.Cu) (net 6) (status 800))
 (segment (start 70.866 48.26) (end 69.85 47.244) (width 0.59944) (layer B.Cu) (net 6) (status 400))
 (segment (start 80.772 48.26) (end 80.772 48.006) (width 0.59944) (layer B.Cu) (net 7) (status 800))
 (segment (start 75.692 46.228) (end 73.66 44.196) (width 0.59944) (layer B.Cu) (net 7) (status 400))
 (segment (start 78.994 46.228) (end 75.692 46.228) (width 0.59944) (layer B.Cu) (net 7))
 (segment (start 80.772 48.006) (end 78.994 46.228) (width 0.59944) (layer B.Cu) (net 7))
 (segment (start 96.774 29.718) (end 96.774 43.688) (width 0.59944) (layer B.Cu) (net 8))
 (segment (start 96.774 43.688) (end 90.678 49.784) (width 0.59944) (layer B.Cu) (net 8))
 (segment (start 88.5317 28.41752) (end 95.47352 28.41752) (width 0.59944) (layer B.Cu) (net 8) (status 800))
 (segment (start 96.774 29.718) (end 95.47352 28.41752) (width 0.59944) (layer B.Cu) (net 8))
 (segment (start 85.852 49.784) (end 90.678 49.784) (width 0.59944) (layer B.Cu) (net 8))
 (segment (start 80.264 44.196) (end 85.852 49.784) (width 0.59944) (layer B.Cu) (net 8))
 (segment (start 80.264 44.196) (end 78.74 44.196) (width 0.59944) (layer B.Cu) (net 8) (status 400))
 (segment (start 43.688 47.752) (end 43.688 46.228) (width 0.59944) (layer B.Cu) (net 9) (status 800))
 (segment (start 43.688 46.228) (end 43.942 45.974) (width 0.59944) (layer B.Cu) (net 9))
 (segment (start 43.942 45.974) (end 45.72 44.196) (width 0.59944) (layer B.Cu) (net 9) (status 400))
 (segment (start 45.72 44.196) (end 44.196 44.196) (width 0.59944) (layer B.Cu) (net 9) (status 800))
 (segment (start 86.868 35.052) (end 86.868 36.322) (width 0.59944) (layer B.Cu) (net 9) (status 400))
 (segment (start 87.884 34.036) (end 86.868 35.052) (width 0.59944) (layer B.Cu) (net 9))
 (segment (start 90.424 34.036) (end 87.884 34.036) (width 0.59944) (layer B.Cu) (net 9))
 (segment (start 91.44 35.052) (end 90.424 34.036) (width 0.59944) (layer B.Cu) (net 9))
 (segment (start 91.44 45.72) (end 91.44 35.052) (width 0.59944) (layer B.Cu) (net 9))
 (segment (start 91.186 45.974) (end 91.44 45.72) (width 0.59944) (layer B.Cu) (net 9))
 (via (at 91.186 45.974) (size 1.143) (layers F.Cu B.Cu) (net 9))
 (segment (start 91.694 45.974) (end 91.186 45.974) (width 0.59944) (layer F.Cu) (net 9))
 (segment (start 42.418 45.974) (end 91.694 45.974) (width 0.59944) (layer F.Cu) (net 9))
 (via (at 42.418 45.974) (size 1.143) (layers F.Cu B.Cu) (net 9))
 (segment (start 44.196 44.196) (end 42.418 45.974) (width 0.59944) (layer B.Cu) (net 9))
 (segment (start 89.408 36.322) (end 89.408 37.084) (width 0.59944) (layer B.Cu) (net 10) (status 800))
 (segment (start 73.66 38.1) (end 73.66 36.576) (width 0.59944) (layer B.Cu) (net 10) (status 400))
 (segment (start 74.422 38.862) (end 73.66 38.1) (width 0.59944) (layer B.Cu) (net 10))
 (segment (start 87.63 38.862) (end 74.422 38.862) (width 0.59944) (layer B.Cu) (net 10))
 (segment (start 89.408 37.084) (end 87.63 38.862) (width 0.59944) (layer B.Cu) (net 10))
 (segment (start 84.328 43.942) (end 84.328 44.958) (width 0.59944) (layer B.Cu) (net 11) (status 800))
 (segment (start 71.12 38.862) (end 71.12 36.576) (width 0.59944) (layer B.Cu) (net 11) (status 400))
 (segment (start 73.152 40.894) (end 71.12 38.862) (width 0.59944) (layer B.Cu) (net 11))
 (segment (start 86.614 40.894) (end 73.152 40.894) (width 0.59944) (layer B.Cu) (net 11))
 (segment (start 88.138 42.418) (end 86.614 40.894) (width 0.59944) (layer B.Cu) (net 11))
 (segment (start 88.138 45.466) (end 88.138 42.418) (width 0.59944) (layer B.Cu) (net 11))
 (segment (start 87.63 45.974) (end 88.138 45.466) (width 0.59944) (layer B.Cu) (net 11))
 (segment (start 85.344 45.974) (end 87.63 45.974) (width 0.59944) (layer B.Cu) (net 11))
 (segment (start 84.328 44.958) (end 85.344 45.974) (width 0.59944) (layer B.Cu) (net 11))
 (segment (start 89.408 43.942) (end 89.408 41.402) (width 0.59944) (layer B.Cu) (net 12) (status 800))
 (segment (start 68.58 35.814) (end 68.58 36.576) (width 0.59944) (layer B.Cu) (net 12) (status 400))
 (segment (start 69.85 34.544) (end 68.58 35.814) (width 0.59944) (layer B.Cu) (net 12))
 (segment (start 71.628 34.544) (end 69.85 34.544) (width 0.59944) (layer B.Cu) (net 12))
 (segment (start 72.39 35.306) (end 71.628 34.544) (width 0.59944) (layer B.Cu) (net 12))
 (segment (start 72.39 38.354) (end 72.39 35.306) (width 0.59944) (layer B.Cu) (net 12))
 (segment (start 73.914 39.878) (end 72.39 38.354) (width 0.59944) (layer B.Cu) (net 12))
 (segment (start 87.884 39.878) (end 73.914 39.878) (width 0.59944) (layer B.Cu) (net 12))
 (segment (start 89.408 41.402) (end 87.884 39.878) (width 0.59944) (layer B.Cu) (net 12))
 (segment (start 80.264 27.178) (end 81.534 27.178) (width 0.59944) (layer B.Cu) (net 13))
 (segment (start 93.59646 30.226) (end 94.94012 31.56966) (width 0.70104) (layer B.Cu) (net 13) (status 400))
 (segment (start 92.964 30.226) (end 93.59646 30.226) (width 0.70104) (layer B.Cu) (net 13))
 (segment (start 82.55 27.178) (end 85.598 30.226) (width 0.59944) (layer B.Cu) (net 13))
 (segment (start 81.534 27.178) (end 82.55 27.178) (width 0.59944) (layer B.Cu) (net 13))
 (segment (start 92.964 30.226) (end 85.598 30.226) (width 0.59944) (layer B.Cu) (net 13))
 (segment (start 80.264 27.178) (end 73.152 27.178) (width 0.59944) (layer B.Cu) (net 13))
 (segment (start 72.39 27.178) (end 73.152 27.178) (width 0.59944) (layer B.Cu) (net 13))
 (segment (start 60.452 27.178) (end 49.784 27.178) (width 0.59944) (layer B.Cu) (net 13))
 (segment (start 48.006 27.178) (end 46.482 28.702) (width 0.59944) (layer B.Cu) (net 13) (status 400))
 (segment (start 49.784 27.178) (end 48.006 27.178) (width 0.59944) (layer B.Cu) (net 13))
 (segment (start 60.452 27.178) (end 72.39 27.178) (width 0.59944) (layer B.Cu) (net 13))
 (segment (start 77.216 32.766) (end 77.216 30.988) (width 0.59944) (layer B.Cu) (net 13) (status 800))
 (segment (start 77.216 30.988) (end 77.47 30.734) (width 0.59944) (layer B.Cu) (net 13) (status 400))
 (segment (start 64.77 33.528) (end 66.04 33.528) (width 0.59944) (layer B.Cu) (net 13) (status 800))
 (segment (start 70.358 29.21) (end 68.58 30.988) (width 0.59944) (layer B.Cu) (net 13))
 (segment (start 71.12 29.21) (end 70.358 29.21) (width 0.59944) (layer B.Cu) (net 13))
 (segment (start 71.12 29.21) (end 72.39 29.21) (width 0.59944) (layer B.Cu) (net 13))
 (segment (start 68.58 30.988) (end 66.04 33.528) (width 0.59944) (layer B.Cu) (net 13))
 (segment (start 80.43164 28.41752) (end 80.43164 27.34564) (width 0.59944) (layer B.Cu) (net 13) (status 800))
 (segment (start 80.43164 27.34564) (end 80.264 27.178) (width 0.59944) (layer B.Cu) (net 13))
 (segment (start 72.39 29.21) (end 72.39 27.178) (width 0.59944) (layer B.Cu) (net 13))
 (segment (start 72.39 29.21) (end 73.406 29.21) (width 0.59944) (layer B.Cu) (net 13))
 (segment (start 74.93 30.734) (end 77.47 30.734) (width 0.59944) (layer B.Cu) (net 13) (status 400))
 (segment (start 73.406 29.21) (end 74.93 30.734) (width 0.59944) (layer B.Cu) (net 13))
 (segment (start 88.392 48.26) (end 90.678 48.26) (width 0.59944) (layer B.Cu) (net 14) (status 800))
 (segment (start 92.71 46.228) (end 92.71 39.878) (width 0.59944) (layer B.Cu) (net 14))
 (segment (start 92.71 39.878) (end 92.71 36.068) (width 0.59944) (layer B.Cu) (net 14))
 (segment (start 92.71 36.068) (end 92.71 33.782) (width 0.59944) (layer B.Cu) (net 14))
 (segment (start 83.566 38.1) (end 79.756 34.29) (width 0.59944) (layer B.Cu) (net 14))
 (segment (start 91.44 32.512) (end 87.63 32.512) (width 0.59944) (layer B.Cu) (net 14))
 (segment (start 87.63 32.512) (end 85.598 34.544) (width 0.59944) (layer B.Cu) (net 14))
 (segment (start 85.598 34.544) (end 85.598 37.338) (width 0.59944) (layer B.Cu) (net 14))
 (segment (start 85.598 37.338) (end 84.836 38.1) (width 0.59944) (layer B.Cu) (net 14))
 (segment (start 84.836 38.1) (end 83.566 38.1) (width 0.59944) (layer B.Cu) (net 14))
 (segment (start 92.71 33.782) (end 91.44 32.512) (width 0.59944) (layer B.Cu) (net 14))
 (segment (start 90.678 48.26) (end 92.71 46.228) (width 0.59944) (layer B.Cu) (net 14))
 (segment (start 75.946 34.29) (end 72.39 30.734) (width 0.59944) (layer B.Cu) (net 14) (status 400))
 (segment (start 79.756 34.29) (end 75.946 34.29) (width 0.59944) (layer B.Cu) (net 14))
 (segment (start 92.71 36.068) (end 94.84106 36.068) (width 0.70104) (layer B.Cu) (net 14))
 (segment (start 94.84106 36.068) (end 94.94012 35.96894) (width 0.70104) (layer B.Cu) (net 14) (status 400))
 (segment (start 57.15 33.528) (end 57.15 33.02) (width 0.59944) (layer B.Cu) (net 15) (status 800))
 (segment (start 57.15 33.02) (end 54.864 30.734) (width 0.59944) (layer B.Cu) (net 15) (status 400))
 (segment (start 54.864 30.734) (end 53.086 28.956) (width 0.59944) (layer B.Cu) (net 15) (status 800))
 (segment (start 49.276 28.956) (end 49.022 28.702) (width 0.59944) (layer B.Cu) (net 15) (status 400))
 (segment (start 53.086 28.956) (end 49.276 28.956) (width 0.59944) (layer B.Cu) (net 15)))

